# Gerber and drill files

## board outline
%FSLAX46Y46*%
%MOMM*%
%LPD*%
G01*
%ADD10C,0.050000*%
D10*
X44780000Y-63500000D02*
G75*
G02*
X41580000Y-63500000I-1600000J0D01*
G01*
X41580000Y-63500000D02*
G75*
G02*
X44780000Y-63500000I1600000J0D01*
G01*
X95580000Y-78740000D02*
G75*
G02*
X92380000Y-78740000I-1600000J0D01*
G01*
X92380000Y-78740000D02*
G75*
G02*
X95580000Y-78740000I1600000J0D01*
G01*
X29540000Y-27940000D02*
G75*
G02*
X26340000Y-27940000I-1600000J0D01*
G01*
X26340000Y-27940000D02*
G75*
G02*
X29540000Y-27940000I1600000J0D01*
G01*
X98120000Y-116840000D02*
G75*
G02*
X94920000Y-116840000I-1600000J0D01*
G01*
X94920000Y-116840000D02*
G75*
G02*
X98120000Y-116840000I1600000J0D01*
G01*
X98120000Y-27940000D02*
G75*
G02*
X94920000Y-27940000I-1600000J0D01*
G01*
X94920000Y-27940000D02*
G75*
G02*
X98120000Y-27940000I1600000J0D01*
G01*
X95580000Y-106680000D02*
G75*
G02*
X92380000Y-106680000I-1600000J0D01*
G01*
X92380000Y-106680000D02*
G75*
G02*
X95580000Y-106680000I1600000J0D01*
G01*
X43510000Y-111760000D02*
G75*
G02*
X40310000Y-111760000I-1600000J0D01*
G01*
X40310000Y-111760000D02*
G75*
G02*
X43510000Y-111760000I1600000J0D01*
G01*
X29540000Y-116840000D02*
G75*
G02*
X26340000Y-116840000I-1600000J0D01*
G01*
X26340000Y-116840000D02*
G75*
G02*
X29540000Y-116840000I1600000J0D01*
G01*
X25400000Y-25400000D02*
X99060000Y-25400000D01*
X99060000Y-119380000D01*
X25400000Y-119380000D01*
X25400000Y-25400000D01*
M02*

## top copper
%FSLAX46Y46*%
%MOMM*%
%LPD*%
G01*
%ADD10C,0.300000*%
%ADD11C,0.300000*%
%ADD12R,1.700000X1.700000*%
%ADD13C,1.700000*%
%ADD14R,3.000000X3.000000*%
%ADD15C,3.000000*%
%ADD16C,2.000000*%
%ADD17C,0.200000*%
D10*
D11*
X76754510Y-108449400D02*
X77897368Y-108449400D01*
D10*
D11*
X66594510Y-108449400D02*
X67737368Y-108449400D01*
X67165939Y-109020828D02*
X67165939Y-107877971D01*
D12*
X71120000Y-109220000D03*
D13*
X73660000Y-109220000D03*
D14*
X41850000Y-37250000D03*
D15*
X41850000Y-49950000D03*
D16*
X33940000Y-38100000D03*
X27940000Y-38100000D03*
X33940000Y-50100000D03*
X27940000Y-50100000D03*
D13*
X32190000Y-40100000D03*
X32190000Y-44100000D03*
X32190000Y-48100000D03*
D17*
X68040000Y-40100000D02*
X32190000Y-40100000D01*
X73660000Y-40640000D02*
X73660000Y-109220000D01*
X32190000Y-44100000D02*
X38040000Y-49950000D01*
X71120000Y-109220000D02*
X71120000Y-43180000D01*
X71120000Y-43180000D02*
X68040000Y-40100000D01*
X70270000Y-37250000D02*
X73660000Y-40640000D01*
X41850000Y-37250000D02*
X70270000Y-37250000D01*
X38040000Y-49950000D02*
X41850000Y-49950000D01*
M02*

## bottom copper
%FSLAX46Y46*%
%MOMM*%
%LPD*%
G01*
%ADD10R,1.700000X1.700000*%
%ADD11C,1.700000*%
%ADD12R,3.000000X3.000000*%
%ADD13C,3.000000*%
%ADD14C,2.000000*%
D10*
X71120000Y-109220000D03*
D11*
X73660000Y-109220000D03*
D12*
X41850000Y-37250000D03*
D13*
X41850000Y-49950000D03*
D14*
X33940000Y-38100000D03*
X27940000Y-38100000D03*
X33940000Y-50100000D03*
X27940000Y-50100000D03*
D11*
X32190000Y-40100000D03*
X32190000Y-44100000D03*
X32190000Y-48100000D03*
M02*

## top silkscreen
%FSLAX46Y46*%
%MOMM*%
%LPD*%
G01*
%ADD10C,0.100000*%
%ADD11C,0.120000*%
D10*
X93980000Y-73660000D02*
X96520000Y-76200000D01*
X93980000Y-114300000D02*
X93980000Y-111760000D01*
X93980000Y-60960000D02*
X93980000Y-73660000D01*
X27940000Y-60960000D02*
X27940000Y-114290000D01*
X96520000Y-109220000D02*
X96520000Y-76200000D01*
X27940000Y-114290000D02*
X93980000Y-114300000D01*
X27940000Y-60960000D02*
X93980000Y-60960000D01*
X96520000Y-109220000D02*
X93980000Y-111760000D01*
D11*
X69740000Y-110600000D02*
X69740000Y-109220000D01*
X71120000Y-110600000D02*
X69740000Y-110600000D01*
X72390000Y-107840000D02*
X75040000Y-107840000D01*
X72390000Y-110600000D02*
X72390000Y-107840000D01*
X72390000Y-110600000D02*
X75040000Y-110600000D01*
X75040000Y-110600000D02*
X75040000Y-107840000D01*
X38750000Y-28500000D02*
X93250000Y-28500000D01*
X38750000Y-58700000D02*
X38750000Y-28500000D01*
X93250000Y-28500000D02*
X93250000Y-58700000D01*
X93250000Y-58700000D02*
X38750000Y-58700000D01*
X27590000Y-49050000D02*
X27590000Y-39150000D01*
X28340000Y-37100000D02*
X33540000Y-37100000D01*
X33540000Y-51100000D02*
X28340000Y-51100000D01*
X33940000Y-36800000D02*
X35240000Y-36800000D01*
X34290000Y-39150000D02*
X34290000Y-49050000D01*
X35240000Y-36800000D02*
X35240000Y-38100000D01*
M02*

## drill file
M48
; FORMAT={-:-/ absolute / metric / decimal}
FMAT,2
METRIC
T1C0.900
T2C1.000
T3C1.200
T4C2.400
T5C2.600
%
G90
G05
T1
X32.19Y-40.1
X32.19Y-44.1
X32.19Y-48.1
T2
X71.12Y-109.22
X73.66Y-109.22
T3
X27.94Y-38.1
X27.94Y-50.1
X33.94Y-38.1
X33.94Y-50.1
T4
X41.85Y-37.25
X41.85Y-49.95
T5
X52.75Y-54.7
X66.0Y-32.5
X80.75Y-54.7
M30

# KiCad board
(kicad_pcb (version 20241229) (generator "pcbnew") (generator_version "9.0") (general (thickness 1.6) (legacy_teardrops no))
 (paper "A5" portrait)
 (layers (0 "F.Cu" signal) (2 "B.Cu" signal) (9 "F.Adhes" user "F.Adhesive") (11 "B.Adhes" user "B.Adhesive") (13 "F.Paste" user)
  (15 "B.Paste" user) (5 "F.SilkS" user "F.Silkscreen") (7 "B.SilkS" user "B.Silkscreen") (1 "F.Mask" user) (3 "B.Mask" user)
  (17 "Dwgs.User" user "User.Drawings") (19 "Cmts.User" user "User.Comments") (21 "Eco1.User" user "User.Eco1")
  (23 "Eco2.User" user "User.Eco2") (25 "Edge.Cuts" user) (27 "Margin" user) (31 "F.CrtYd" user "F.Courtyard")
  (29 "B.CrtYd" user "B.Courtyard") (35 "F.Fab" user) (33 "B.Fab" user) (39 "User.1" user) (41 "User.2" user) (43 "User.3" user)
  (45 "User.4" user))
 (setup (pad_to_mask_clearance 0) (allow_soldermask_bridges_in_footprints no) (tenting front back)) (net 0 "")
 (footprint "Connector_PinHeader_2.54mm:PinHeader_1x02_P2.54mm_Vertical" (layer "F.Cu") (at 71.12 109.22 90)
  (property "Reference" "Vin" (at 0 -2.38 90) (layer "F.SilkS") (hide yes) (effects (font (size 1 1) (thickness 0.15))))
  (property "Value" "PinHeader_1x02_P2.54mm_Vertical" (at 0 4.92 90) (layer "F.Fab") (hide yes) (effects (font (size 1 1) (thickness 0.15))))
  (fp_line (start -1.38 -1.38) (end 0 -1.38) (stroke (width 0.12) (type solid)) (layer "F.SilkS"))
  (fp_line (start -1.38 0) (end -1.38 -1.38) (stroke (width 0.12) (type solid)) (layer "F.SilkS"))
  (fp_line (start 1.38 1.27) (end 1.38 3.92) (stroke (width 0.12) (type solid)) (layer "F.SilkS"))
  (fp_line (start -1.38 1.27) (end 1.38 1.27) (stroke (width 0.12) (type solid)) (layer "F.SilkS"))
  (fp_line (start -1.38 1.27) (end -1.38 3.92) (stroke (width 0.12) (type solid)) (layer "F.SilkS"))
  (fp_line (start -1.38 3.92) (end 1.38 3.92) (stroke (width 0.12) (type solid)) (layer "F.SilkS"))
  (pad "1" thru_hole rect (at 0 0 90) (size 1.7 1.7) (drill 1) (layers "*.Cu" "*.Mask") (remove_unused_layers no))
  (pad "2" thru_hole circle (at 0 2.54 90) (size 1.7 1.7) (drill 1) (layers "*.Cu" "*.Mask") (remove_unused_layers no)))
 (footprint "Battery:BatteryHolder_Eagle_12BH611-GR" (layer "F.Cu") (at 41.85 37.25 180)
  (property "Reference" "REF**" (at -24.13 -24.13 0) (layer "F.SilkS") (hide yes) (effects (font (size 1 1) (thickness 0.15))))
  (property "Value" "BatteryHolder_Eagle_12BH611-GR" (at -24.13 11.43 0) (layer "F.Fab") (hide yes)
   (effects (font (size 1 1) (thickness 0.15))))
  (fp_line (start 3.1 8.75) (end -51.4 8.75) (stroke (width 0.12) (type solid)) (layer "F.SilkS"))
  (fp_line (start 3.1 -21.45) (end 3.1 8.75) (stroke (width 0.12) (type solid)) (layer "F.SilkS"))
  (fp_line (start -51.4 8.75) (end -51.4 -21.45) (stroke (width 0.12) (type solid)) (layer "F.SilkS"))
  (fp_line (start -51.4 -21.45) (end 3.1 -21.45) (stroke (width 0.12) (type solid)) (layer "F.SilkS"))
  (pad "" np_thru_hole circle (at -38.9 -17.45 180) (size 2.6 2.6) (drill 2.6) (layers "*.Cu" "*.Mask"))
  (pad "" np_thru_hole circle (at -24.15 4.75 180) (size 2.6 2.6) (drill 2.6) (layers "*.Cu" "*.Mask"))
  (pad "" np_thru_hole circle (at -10.9 -17.45 180) (size 2.6 2.6) (drill 2.6) (layers "*.Cu" "*.Mask"))
  (pad "1" thru_hole rect (at 0 0 180) (size 3 3) (drill 2.4) (layers "*.Cu" "*.Mask") (remove_unused_layers no))
  (pad "2" thru_hole circle (at 0 -12.7 180) (size 3 3) (drill 2.4) (layers "*.Cu" "*.Mask") (remove_unused_layers no)))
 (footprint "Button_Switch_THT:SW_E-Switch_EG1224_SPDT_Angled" (layer "F.Cu") (at 32.19 40.1 -90)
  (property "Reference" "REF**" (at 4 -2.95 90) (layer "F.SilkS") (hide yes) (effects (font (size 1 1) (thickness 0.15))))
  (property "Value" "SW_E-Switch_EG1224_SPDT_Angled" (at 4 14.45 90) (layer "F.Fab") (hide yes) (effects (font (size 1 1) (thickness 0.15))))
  (fp_line (start 8.95 4.6) (end -0.95 4.6) (stroke (width 0.12) (type solid)) (layer "F.SilkS"))
  (fp_line (start -3 3.85) (end -3 -1.35) (stroke (width 0.12) (type solid)) (layer "F.SilkS"))
  (fp_line (start 11 -1.35) (end 11 3.85) (stroke (width 0.12) (type solid)) (layer "F.SilkS"))
  (fp_line (start -3.3 -1.75) (end -3.3 -3.05) (stroke (width 0.12) (type solid)) (layer "F.SilkS"))
  (fp_line (start -0.95 -2.1) (end 8.95 -2.1) (stroke (width 0.12) (type solid)) (layer "F.SilkS"))
  (fp_line (start -3.3 -3.05) (end -2 -3.05) (stroke (width 0.12) (type solid)) (layer "F.SilkS"))
  (pad "" thru_hole circle (at -2 -1.75 270) (size 2 2) (drill 1.2) (layers "*.Cu" "*.Mask") (remove_unused_layers no))
  (pad "" thru_hole circle (at -2 4.25 270) (size 2 2) (drill 1.2) (layers "*.Cu" "*.Mask") (remove_unused_layers no))
  (pad "" thru_hole circle (at 10 -1.75 270) (size 2 2) (drill 1.2) (layers "*.Cu" "*.Mask") (remove_unused_layers no))
  (pad "" thru_hole circle (at 10 4.25 270) (size 2 2) (drill 1.2) (layers "*.Cu" "*.Mask") (remove_unused_layers no))
  (pad "1" thru_hole circle (at 0 0 270) (size 1.7 1.7) (drill 0.9) (layers "*.Cu" "*.Mask") (remove_unused_layers no))
  (pad "2" thru_hole circle (at 4 0 270) (size 1.7 1.7) (drill 0.9) (layers "*.Cu" "*.Mask") (remove_unused_layers no))
  (pad "3" thru_hole circle (at 8 0 270) (size 1.7 1.7) (drill 0.9) (layers "*.Cu" "*.Mask") (remove_unused_layers no)))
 (gr_line (start 93.98 73.66) (end 96.52 76.2) (stroke (width 0.1) (type solid)) (layer "F.SilkS"))
 (gr_line (start 93.98 114.3) (end 93.98 111.76) (stroke (width 0.1) (type solid)) (layer "F.SilkS"))
 (gr_line (start 93.98 60.96) (end 93.98 73.66) (stroke (width 0.1) (type solid)) (layer "F.SilkS"))
 (gr_line (start 27.94 60.96) (end 27.94 114.29) (stroke (width 0.1) (type solid)) (layer "F.SilkS"))
 (gr_line (start 96.52 109.22) (end 96.52 76.2) (stroke (width 0.1) (type solid)) (layer "F.SilkS"))
 (gr_line (start 27.94 114.29) (end 93.98 114.3) (stroke (width 0.1) (type solid)) (layer "F.SilkS"))
 (gr_line (start 27.94 60.96) (end 93.98 60.96) (stroke (width 0.1) (type solid)) (layer "F.SilkS"))
 (gr_line (start 96.52 109.22) (end 93.98 111.76) (stroke (width 0.1) (type default)) (layer "F.SilkS"))
 (gr_circle (center 43.18 63.5) (end 44.78 63.5) (stroke (width 0.05) (type solid)) (fill no) (layer "Edge.Cuts"))
 (gr_circle (center 93.98 78.74) (end 95.58 78.74) (stroke (width 0.05) (type solid)) (fill no) (layer "Edge.Cuts"))
 (gr_circle (center 27.94 27.94) (end 29.54 27.94) (stroke (width 0.05) (type solid)) (fill no) (layer "Edge.Cuts"))
 (gr_circle (center 96.52 116.84) (end 98.12 116.84) (stroke (width 0.05) (type solid)) (fill no) (layer "Edge.Cuts"))
 (gr_circle (center 96.52 27.94) (end 98.12 27.94) (stroke (width 0.05) (type solid)) (fill no) (layer "Edge.Cuts"))
 (gr_circle (center 93.98 106.68) (end 95.58 106.68) (stroke (width 0.05) (type solid)) (fill no) (layer "Edge.Cuts"))
 (gr_circle (center 41.91 111.76) (end 43.51 111.76) (stroke (width 0.05) (type solid)) (fill no) (layer "Edge.Cuts"))
 (gr_circle (center 27.94 116.84) (end 29.54 116.84) (stroke (width 0.05) (type solid)) (fill no) (layer "Edge.Cuts"))
 (gr_rect (start 25.4 25.4) (end 99.06 119.38) (stroke (width 0.05) (type default)) (fill no) (layer "Edge.Cuts"))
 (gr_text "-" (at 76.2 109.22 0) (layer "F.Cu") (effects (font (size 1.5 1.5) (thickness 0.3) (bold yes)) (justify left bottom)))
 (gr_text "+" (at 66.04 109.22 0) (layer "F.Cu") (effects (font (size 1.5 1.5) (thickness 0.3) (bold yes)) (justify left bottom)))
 (segment (start 68.04 40.1) (end 32.19 40.1) (width 0.2) (layer "F.Cu") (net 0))
 (segment (start 73.66 40.64) (end 73.66 109.22) (width 0.2) (layer "F.Cu") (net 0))
 (segment (start 32.19 44.1) (end 38.04 49.95) (width 0.2) (layer "F.Cu") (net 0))
 (segment (start 71.12 109.22) (end 71.12 43.18) (width 0.2) (layer "F.Cu") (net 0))
 (segment (start 71.12 43.18) (end 68.04 40.1) (width 0.2) (layer "F.Cu") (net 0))
 (segment (start 70.27 37.25) (end 73.66 40.64) (width 0.2) (layer "F.Cu") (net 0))
 (segment (start 41.85 37.25) (end 70.27 37.25) (width 0.2) (layer "F.Cu") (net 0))
 (segment (start 38.04 49.95) (end 41.85 49.95) (width 0.2) (layer "F.Cu") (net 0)))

